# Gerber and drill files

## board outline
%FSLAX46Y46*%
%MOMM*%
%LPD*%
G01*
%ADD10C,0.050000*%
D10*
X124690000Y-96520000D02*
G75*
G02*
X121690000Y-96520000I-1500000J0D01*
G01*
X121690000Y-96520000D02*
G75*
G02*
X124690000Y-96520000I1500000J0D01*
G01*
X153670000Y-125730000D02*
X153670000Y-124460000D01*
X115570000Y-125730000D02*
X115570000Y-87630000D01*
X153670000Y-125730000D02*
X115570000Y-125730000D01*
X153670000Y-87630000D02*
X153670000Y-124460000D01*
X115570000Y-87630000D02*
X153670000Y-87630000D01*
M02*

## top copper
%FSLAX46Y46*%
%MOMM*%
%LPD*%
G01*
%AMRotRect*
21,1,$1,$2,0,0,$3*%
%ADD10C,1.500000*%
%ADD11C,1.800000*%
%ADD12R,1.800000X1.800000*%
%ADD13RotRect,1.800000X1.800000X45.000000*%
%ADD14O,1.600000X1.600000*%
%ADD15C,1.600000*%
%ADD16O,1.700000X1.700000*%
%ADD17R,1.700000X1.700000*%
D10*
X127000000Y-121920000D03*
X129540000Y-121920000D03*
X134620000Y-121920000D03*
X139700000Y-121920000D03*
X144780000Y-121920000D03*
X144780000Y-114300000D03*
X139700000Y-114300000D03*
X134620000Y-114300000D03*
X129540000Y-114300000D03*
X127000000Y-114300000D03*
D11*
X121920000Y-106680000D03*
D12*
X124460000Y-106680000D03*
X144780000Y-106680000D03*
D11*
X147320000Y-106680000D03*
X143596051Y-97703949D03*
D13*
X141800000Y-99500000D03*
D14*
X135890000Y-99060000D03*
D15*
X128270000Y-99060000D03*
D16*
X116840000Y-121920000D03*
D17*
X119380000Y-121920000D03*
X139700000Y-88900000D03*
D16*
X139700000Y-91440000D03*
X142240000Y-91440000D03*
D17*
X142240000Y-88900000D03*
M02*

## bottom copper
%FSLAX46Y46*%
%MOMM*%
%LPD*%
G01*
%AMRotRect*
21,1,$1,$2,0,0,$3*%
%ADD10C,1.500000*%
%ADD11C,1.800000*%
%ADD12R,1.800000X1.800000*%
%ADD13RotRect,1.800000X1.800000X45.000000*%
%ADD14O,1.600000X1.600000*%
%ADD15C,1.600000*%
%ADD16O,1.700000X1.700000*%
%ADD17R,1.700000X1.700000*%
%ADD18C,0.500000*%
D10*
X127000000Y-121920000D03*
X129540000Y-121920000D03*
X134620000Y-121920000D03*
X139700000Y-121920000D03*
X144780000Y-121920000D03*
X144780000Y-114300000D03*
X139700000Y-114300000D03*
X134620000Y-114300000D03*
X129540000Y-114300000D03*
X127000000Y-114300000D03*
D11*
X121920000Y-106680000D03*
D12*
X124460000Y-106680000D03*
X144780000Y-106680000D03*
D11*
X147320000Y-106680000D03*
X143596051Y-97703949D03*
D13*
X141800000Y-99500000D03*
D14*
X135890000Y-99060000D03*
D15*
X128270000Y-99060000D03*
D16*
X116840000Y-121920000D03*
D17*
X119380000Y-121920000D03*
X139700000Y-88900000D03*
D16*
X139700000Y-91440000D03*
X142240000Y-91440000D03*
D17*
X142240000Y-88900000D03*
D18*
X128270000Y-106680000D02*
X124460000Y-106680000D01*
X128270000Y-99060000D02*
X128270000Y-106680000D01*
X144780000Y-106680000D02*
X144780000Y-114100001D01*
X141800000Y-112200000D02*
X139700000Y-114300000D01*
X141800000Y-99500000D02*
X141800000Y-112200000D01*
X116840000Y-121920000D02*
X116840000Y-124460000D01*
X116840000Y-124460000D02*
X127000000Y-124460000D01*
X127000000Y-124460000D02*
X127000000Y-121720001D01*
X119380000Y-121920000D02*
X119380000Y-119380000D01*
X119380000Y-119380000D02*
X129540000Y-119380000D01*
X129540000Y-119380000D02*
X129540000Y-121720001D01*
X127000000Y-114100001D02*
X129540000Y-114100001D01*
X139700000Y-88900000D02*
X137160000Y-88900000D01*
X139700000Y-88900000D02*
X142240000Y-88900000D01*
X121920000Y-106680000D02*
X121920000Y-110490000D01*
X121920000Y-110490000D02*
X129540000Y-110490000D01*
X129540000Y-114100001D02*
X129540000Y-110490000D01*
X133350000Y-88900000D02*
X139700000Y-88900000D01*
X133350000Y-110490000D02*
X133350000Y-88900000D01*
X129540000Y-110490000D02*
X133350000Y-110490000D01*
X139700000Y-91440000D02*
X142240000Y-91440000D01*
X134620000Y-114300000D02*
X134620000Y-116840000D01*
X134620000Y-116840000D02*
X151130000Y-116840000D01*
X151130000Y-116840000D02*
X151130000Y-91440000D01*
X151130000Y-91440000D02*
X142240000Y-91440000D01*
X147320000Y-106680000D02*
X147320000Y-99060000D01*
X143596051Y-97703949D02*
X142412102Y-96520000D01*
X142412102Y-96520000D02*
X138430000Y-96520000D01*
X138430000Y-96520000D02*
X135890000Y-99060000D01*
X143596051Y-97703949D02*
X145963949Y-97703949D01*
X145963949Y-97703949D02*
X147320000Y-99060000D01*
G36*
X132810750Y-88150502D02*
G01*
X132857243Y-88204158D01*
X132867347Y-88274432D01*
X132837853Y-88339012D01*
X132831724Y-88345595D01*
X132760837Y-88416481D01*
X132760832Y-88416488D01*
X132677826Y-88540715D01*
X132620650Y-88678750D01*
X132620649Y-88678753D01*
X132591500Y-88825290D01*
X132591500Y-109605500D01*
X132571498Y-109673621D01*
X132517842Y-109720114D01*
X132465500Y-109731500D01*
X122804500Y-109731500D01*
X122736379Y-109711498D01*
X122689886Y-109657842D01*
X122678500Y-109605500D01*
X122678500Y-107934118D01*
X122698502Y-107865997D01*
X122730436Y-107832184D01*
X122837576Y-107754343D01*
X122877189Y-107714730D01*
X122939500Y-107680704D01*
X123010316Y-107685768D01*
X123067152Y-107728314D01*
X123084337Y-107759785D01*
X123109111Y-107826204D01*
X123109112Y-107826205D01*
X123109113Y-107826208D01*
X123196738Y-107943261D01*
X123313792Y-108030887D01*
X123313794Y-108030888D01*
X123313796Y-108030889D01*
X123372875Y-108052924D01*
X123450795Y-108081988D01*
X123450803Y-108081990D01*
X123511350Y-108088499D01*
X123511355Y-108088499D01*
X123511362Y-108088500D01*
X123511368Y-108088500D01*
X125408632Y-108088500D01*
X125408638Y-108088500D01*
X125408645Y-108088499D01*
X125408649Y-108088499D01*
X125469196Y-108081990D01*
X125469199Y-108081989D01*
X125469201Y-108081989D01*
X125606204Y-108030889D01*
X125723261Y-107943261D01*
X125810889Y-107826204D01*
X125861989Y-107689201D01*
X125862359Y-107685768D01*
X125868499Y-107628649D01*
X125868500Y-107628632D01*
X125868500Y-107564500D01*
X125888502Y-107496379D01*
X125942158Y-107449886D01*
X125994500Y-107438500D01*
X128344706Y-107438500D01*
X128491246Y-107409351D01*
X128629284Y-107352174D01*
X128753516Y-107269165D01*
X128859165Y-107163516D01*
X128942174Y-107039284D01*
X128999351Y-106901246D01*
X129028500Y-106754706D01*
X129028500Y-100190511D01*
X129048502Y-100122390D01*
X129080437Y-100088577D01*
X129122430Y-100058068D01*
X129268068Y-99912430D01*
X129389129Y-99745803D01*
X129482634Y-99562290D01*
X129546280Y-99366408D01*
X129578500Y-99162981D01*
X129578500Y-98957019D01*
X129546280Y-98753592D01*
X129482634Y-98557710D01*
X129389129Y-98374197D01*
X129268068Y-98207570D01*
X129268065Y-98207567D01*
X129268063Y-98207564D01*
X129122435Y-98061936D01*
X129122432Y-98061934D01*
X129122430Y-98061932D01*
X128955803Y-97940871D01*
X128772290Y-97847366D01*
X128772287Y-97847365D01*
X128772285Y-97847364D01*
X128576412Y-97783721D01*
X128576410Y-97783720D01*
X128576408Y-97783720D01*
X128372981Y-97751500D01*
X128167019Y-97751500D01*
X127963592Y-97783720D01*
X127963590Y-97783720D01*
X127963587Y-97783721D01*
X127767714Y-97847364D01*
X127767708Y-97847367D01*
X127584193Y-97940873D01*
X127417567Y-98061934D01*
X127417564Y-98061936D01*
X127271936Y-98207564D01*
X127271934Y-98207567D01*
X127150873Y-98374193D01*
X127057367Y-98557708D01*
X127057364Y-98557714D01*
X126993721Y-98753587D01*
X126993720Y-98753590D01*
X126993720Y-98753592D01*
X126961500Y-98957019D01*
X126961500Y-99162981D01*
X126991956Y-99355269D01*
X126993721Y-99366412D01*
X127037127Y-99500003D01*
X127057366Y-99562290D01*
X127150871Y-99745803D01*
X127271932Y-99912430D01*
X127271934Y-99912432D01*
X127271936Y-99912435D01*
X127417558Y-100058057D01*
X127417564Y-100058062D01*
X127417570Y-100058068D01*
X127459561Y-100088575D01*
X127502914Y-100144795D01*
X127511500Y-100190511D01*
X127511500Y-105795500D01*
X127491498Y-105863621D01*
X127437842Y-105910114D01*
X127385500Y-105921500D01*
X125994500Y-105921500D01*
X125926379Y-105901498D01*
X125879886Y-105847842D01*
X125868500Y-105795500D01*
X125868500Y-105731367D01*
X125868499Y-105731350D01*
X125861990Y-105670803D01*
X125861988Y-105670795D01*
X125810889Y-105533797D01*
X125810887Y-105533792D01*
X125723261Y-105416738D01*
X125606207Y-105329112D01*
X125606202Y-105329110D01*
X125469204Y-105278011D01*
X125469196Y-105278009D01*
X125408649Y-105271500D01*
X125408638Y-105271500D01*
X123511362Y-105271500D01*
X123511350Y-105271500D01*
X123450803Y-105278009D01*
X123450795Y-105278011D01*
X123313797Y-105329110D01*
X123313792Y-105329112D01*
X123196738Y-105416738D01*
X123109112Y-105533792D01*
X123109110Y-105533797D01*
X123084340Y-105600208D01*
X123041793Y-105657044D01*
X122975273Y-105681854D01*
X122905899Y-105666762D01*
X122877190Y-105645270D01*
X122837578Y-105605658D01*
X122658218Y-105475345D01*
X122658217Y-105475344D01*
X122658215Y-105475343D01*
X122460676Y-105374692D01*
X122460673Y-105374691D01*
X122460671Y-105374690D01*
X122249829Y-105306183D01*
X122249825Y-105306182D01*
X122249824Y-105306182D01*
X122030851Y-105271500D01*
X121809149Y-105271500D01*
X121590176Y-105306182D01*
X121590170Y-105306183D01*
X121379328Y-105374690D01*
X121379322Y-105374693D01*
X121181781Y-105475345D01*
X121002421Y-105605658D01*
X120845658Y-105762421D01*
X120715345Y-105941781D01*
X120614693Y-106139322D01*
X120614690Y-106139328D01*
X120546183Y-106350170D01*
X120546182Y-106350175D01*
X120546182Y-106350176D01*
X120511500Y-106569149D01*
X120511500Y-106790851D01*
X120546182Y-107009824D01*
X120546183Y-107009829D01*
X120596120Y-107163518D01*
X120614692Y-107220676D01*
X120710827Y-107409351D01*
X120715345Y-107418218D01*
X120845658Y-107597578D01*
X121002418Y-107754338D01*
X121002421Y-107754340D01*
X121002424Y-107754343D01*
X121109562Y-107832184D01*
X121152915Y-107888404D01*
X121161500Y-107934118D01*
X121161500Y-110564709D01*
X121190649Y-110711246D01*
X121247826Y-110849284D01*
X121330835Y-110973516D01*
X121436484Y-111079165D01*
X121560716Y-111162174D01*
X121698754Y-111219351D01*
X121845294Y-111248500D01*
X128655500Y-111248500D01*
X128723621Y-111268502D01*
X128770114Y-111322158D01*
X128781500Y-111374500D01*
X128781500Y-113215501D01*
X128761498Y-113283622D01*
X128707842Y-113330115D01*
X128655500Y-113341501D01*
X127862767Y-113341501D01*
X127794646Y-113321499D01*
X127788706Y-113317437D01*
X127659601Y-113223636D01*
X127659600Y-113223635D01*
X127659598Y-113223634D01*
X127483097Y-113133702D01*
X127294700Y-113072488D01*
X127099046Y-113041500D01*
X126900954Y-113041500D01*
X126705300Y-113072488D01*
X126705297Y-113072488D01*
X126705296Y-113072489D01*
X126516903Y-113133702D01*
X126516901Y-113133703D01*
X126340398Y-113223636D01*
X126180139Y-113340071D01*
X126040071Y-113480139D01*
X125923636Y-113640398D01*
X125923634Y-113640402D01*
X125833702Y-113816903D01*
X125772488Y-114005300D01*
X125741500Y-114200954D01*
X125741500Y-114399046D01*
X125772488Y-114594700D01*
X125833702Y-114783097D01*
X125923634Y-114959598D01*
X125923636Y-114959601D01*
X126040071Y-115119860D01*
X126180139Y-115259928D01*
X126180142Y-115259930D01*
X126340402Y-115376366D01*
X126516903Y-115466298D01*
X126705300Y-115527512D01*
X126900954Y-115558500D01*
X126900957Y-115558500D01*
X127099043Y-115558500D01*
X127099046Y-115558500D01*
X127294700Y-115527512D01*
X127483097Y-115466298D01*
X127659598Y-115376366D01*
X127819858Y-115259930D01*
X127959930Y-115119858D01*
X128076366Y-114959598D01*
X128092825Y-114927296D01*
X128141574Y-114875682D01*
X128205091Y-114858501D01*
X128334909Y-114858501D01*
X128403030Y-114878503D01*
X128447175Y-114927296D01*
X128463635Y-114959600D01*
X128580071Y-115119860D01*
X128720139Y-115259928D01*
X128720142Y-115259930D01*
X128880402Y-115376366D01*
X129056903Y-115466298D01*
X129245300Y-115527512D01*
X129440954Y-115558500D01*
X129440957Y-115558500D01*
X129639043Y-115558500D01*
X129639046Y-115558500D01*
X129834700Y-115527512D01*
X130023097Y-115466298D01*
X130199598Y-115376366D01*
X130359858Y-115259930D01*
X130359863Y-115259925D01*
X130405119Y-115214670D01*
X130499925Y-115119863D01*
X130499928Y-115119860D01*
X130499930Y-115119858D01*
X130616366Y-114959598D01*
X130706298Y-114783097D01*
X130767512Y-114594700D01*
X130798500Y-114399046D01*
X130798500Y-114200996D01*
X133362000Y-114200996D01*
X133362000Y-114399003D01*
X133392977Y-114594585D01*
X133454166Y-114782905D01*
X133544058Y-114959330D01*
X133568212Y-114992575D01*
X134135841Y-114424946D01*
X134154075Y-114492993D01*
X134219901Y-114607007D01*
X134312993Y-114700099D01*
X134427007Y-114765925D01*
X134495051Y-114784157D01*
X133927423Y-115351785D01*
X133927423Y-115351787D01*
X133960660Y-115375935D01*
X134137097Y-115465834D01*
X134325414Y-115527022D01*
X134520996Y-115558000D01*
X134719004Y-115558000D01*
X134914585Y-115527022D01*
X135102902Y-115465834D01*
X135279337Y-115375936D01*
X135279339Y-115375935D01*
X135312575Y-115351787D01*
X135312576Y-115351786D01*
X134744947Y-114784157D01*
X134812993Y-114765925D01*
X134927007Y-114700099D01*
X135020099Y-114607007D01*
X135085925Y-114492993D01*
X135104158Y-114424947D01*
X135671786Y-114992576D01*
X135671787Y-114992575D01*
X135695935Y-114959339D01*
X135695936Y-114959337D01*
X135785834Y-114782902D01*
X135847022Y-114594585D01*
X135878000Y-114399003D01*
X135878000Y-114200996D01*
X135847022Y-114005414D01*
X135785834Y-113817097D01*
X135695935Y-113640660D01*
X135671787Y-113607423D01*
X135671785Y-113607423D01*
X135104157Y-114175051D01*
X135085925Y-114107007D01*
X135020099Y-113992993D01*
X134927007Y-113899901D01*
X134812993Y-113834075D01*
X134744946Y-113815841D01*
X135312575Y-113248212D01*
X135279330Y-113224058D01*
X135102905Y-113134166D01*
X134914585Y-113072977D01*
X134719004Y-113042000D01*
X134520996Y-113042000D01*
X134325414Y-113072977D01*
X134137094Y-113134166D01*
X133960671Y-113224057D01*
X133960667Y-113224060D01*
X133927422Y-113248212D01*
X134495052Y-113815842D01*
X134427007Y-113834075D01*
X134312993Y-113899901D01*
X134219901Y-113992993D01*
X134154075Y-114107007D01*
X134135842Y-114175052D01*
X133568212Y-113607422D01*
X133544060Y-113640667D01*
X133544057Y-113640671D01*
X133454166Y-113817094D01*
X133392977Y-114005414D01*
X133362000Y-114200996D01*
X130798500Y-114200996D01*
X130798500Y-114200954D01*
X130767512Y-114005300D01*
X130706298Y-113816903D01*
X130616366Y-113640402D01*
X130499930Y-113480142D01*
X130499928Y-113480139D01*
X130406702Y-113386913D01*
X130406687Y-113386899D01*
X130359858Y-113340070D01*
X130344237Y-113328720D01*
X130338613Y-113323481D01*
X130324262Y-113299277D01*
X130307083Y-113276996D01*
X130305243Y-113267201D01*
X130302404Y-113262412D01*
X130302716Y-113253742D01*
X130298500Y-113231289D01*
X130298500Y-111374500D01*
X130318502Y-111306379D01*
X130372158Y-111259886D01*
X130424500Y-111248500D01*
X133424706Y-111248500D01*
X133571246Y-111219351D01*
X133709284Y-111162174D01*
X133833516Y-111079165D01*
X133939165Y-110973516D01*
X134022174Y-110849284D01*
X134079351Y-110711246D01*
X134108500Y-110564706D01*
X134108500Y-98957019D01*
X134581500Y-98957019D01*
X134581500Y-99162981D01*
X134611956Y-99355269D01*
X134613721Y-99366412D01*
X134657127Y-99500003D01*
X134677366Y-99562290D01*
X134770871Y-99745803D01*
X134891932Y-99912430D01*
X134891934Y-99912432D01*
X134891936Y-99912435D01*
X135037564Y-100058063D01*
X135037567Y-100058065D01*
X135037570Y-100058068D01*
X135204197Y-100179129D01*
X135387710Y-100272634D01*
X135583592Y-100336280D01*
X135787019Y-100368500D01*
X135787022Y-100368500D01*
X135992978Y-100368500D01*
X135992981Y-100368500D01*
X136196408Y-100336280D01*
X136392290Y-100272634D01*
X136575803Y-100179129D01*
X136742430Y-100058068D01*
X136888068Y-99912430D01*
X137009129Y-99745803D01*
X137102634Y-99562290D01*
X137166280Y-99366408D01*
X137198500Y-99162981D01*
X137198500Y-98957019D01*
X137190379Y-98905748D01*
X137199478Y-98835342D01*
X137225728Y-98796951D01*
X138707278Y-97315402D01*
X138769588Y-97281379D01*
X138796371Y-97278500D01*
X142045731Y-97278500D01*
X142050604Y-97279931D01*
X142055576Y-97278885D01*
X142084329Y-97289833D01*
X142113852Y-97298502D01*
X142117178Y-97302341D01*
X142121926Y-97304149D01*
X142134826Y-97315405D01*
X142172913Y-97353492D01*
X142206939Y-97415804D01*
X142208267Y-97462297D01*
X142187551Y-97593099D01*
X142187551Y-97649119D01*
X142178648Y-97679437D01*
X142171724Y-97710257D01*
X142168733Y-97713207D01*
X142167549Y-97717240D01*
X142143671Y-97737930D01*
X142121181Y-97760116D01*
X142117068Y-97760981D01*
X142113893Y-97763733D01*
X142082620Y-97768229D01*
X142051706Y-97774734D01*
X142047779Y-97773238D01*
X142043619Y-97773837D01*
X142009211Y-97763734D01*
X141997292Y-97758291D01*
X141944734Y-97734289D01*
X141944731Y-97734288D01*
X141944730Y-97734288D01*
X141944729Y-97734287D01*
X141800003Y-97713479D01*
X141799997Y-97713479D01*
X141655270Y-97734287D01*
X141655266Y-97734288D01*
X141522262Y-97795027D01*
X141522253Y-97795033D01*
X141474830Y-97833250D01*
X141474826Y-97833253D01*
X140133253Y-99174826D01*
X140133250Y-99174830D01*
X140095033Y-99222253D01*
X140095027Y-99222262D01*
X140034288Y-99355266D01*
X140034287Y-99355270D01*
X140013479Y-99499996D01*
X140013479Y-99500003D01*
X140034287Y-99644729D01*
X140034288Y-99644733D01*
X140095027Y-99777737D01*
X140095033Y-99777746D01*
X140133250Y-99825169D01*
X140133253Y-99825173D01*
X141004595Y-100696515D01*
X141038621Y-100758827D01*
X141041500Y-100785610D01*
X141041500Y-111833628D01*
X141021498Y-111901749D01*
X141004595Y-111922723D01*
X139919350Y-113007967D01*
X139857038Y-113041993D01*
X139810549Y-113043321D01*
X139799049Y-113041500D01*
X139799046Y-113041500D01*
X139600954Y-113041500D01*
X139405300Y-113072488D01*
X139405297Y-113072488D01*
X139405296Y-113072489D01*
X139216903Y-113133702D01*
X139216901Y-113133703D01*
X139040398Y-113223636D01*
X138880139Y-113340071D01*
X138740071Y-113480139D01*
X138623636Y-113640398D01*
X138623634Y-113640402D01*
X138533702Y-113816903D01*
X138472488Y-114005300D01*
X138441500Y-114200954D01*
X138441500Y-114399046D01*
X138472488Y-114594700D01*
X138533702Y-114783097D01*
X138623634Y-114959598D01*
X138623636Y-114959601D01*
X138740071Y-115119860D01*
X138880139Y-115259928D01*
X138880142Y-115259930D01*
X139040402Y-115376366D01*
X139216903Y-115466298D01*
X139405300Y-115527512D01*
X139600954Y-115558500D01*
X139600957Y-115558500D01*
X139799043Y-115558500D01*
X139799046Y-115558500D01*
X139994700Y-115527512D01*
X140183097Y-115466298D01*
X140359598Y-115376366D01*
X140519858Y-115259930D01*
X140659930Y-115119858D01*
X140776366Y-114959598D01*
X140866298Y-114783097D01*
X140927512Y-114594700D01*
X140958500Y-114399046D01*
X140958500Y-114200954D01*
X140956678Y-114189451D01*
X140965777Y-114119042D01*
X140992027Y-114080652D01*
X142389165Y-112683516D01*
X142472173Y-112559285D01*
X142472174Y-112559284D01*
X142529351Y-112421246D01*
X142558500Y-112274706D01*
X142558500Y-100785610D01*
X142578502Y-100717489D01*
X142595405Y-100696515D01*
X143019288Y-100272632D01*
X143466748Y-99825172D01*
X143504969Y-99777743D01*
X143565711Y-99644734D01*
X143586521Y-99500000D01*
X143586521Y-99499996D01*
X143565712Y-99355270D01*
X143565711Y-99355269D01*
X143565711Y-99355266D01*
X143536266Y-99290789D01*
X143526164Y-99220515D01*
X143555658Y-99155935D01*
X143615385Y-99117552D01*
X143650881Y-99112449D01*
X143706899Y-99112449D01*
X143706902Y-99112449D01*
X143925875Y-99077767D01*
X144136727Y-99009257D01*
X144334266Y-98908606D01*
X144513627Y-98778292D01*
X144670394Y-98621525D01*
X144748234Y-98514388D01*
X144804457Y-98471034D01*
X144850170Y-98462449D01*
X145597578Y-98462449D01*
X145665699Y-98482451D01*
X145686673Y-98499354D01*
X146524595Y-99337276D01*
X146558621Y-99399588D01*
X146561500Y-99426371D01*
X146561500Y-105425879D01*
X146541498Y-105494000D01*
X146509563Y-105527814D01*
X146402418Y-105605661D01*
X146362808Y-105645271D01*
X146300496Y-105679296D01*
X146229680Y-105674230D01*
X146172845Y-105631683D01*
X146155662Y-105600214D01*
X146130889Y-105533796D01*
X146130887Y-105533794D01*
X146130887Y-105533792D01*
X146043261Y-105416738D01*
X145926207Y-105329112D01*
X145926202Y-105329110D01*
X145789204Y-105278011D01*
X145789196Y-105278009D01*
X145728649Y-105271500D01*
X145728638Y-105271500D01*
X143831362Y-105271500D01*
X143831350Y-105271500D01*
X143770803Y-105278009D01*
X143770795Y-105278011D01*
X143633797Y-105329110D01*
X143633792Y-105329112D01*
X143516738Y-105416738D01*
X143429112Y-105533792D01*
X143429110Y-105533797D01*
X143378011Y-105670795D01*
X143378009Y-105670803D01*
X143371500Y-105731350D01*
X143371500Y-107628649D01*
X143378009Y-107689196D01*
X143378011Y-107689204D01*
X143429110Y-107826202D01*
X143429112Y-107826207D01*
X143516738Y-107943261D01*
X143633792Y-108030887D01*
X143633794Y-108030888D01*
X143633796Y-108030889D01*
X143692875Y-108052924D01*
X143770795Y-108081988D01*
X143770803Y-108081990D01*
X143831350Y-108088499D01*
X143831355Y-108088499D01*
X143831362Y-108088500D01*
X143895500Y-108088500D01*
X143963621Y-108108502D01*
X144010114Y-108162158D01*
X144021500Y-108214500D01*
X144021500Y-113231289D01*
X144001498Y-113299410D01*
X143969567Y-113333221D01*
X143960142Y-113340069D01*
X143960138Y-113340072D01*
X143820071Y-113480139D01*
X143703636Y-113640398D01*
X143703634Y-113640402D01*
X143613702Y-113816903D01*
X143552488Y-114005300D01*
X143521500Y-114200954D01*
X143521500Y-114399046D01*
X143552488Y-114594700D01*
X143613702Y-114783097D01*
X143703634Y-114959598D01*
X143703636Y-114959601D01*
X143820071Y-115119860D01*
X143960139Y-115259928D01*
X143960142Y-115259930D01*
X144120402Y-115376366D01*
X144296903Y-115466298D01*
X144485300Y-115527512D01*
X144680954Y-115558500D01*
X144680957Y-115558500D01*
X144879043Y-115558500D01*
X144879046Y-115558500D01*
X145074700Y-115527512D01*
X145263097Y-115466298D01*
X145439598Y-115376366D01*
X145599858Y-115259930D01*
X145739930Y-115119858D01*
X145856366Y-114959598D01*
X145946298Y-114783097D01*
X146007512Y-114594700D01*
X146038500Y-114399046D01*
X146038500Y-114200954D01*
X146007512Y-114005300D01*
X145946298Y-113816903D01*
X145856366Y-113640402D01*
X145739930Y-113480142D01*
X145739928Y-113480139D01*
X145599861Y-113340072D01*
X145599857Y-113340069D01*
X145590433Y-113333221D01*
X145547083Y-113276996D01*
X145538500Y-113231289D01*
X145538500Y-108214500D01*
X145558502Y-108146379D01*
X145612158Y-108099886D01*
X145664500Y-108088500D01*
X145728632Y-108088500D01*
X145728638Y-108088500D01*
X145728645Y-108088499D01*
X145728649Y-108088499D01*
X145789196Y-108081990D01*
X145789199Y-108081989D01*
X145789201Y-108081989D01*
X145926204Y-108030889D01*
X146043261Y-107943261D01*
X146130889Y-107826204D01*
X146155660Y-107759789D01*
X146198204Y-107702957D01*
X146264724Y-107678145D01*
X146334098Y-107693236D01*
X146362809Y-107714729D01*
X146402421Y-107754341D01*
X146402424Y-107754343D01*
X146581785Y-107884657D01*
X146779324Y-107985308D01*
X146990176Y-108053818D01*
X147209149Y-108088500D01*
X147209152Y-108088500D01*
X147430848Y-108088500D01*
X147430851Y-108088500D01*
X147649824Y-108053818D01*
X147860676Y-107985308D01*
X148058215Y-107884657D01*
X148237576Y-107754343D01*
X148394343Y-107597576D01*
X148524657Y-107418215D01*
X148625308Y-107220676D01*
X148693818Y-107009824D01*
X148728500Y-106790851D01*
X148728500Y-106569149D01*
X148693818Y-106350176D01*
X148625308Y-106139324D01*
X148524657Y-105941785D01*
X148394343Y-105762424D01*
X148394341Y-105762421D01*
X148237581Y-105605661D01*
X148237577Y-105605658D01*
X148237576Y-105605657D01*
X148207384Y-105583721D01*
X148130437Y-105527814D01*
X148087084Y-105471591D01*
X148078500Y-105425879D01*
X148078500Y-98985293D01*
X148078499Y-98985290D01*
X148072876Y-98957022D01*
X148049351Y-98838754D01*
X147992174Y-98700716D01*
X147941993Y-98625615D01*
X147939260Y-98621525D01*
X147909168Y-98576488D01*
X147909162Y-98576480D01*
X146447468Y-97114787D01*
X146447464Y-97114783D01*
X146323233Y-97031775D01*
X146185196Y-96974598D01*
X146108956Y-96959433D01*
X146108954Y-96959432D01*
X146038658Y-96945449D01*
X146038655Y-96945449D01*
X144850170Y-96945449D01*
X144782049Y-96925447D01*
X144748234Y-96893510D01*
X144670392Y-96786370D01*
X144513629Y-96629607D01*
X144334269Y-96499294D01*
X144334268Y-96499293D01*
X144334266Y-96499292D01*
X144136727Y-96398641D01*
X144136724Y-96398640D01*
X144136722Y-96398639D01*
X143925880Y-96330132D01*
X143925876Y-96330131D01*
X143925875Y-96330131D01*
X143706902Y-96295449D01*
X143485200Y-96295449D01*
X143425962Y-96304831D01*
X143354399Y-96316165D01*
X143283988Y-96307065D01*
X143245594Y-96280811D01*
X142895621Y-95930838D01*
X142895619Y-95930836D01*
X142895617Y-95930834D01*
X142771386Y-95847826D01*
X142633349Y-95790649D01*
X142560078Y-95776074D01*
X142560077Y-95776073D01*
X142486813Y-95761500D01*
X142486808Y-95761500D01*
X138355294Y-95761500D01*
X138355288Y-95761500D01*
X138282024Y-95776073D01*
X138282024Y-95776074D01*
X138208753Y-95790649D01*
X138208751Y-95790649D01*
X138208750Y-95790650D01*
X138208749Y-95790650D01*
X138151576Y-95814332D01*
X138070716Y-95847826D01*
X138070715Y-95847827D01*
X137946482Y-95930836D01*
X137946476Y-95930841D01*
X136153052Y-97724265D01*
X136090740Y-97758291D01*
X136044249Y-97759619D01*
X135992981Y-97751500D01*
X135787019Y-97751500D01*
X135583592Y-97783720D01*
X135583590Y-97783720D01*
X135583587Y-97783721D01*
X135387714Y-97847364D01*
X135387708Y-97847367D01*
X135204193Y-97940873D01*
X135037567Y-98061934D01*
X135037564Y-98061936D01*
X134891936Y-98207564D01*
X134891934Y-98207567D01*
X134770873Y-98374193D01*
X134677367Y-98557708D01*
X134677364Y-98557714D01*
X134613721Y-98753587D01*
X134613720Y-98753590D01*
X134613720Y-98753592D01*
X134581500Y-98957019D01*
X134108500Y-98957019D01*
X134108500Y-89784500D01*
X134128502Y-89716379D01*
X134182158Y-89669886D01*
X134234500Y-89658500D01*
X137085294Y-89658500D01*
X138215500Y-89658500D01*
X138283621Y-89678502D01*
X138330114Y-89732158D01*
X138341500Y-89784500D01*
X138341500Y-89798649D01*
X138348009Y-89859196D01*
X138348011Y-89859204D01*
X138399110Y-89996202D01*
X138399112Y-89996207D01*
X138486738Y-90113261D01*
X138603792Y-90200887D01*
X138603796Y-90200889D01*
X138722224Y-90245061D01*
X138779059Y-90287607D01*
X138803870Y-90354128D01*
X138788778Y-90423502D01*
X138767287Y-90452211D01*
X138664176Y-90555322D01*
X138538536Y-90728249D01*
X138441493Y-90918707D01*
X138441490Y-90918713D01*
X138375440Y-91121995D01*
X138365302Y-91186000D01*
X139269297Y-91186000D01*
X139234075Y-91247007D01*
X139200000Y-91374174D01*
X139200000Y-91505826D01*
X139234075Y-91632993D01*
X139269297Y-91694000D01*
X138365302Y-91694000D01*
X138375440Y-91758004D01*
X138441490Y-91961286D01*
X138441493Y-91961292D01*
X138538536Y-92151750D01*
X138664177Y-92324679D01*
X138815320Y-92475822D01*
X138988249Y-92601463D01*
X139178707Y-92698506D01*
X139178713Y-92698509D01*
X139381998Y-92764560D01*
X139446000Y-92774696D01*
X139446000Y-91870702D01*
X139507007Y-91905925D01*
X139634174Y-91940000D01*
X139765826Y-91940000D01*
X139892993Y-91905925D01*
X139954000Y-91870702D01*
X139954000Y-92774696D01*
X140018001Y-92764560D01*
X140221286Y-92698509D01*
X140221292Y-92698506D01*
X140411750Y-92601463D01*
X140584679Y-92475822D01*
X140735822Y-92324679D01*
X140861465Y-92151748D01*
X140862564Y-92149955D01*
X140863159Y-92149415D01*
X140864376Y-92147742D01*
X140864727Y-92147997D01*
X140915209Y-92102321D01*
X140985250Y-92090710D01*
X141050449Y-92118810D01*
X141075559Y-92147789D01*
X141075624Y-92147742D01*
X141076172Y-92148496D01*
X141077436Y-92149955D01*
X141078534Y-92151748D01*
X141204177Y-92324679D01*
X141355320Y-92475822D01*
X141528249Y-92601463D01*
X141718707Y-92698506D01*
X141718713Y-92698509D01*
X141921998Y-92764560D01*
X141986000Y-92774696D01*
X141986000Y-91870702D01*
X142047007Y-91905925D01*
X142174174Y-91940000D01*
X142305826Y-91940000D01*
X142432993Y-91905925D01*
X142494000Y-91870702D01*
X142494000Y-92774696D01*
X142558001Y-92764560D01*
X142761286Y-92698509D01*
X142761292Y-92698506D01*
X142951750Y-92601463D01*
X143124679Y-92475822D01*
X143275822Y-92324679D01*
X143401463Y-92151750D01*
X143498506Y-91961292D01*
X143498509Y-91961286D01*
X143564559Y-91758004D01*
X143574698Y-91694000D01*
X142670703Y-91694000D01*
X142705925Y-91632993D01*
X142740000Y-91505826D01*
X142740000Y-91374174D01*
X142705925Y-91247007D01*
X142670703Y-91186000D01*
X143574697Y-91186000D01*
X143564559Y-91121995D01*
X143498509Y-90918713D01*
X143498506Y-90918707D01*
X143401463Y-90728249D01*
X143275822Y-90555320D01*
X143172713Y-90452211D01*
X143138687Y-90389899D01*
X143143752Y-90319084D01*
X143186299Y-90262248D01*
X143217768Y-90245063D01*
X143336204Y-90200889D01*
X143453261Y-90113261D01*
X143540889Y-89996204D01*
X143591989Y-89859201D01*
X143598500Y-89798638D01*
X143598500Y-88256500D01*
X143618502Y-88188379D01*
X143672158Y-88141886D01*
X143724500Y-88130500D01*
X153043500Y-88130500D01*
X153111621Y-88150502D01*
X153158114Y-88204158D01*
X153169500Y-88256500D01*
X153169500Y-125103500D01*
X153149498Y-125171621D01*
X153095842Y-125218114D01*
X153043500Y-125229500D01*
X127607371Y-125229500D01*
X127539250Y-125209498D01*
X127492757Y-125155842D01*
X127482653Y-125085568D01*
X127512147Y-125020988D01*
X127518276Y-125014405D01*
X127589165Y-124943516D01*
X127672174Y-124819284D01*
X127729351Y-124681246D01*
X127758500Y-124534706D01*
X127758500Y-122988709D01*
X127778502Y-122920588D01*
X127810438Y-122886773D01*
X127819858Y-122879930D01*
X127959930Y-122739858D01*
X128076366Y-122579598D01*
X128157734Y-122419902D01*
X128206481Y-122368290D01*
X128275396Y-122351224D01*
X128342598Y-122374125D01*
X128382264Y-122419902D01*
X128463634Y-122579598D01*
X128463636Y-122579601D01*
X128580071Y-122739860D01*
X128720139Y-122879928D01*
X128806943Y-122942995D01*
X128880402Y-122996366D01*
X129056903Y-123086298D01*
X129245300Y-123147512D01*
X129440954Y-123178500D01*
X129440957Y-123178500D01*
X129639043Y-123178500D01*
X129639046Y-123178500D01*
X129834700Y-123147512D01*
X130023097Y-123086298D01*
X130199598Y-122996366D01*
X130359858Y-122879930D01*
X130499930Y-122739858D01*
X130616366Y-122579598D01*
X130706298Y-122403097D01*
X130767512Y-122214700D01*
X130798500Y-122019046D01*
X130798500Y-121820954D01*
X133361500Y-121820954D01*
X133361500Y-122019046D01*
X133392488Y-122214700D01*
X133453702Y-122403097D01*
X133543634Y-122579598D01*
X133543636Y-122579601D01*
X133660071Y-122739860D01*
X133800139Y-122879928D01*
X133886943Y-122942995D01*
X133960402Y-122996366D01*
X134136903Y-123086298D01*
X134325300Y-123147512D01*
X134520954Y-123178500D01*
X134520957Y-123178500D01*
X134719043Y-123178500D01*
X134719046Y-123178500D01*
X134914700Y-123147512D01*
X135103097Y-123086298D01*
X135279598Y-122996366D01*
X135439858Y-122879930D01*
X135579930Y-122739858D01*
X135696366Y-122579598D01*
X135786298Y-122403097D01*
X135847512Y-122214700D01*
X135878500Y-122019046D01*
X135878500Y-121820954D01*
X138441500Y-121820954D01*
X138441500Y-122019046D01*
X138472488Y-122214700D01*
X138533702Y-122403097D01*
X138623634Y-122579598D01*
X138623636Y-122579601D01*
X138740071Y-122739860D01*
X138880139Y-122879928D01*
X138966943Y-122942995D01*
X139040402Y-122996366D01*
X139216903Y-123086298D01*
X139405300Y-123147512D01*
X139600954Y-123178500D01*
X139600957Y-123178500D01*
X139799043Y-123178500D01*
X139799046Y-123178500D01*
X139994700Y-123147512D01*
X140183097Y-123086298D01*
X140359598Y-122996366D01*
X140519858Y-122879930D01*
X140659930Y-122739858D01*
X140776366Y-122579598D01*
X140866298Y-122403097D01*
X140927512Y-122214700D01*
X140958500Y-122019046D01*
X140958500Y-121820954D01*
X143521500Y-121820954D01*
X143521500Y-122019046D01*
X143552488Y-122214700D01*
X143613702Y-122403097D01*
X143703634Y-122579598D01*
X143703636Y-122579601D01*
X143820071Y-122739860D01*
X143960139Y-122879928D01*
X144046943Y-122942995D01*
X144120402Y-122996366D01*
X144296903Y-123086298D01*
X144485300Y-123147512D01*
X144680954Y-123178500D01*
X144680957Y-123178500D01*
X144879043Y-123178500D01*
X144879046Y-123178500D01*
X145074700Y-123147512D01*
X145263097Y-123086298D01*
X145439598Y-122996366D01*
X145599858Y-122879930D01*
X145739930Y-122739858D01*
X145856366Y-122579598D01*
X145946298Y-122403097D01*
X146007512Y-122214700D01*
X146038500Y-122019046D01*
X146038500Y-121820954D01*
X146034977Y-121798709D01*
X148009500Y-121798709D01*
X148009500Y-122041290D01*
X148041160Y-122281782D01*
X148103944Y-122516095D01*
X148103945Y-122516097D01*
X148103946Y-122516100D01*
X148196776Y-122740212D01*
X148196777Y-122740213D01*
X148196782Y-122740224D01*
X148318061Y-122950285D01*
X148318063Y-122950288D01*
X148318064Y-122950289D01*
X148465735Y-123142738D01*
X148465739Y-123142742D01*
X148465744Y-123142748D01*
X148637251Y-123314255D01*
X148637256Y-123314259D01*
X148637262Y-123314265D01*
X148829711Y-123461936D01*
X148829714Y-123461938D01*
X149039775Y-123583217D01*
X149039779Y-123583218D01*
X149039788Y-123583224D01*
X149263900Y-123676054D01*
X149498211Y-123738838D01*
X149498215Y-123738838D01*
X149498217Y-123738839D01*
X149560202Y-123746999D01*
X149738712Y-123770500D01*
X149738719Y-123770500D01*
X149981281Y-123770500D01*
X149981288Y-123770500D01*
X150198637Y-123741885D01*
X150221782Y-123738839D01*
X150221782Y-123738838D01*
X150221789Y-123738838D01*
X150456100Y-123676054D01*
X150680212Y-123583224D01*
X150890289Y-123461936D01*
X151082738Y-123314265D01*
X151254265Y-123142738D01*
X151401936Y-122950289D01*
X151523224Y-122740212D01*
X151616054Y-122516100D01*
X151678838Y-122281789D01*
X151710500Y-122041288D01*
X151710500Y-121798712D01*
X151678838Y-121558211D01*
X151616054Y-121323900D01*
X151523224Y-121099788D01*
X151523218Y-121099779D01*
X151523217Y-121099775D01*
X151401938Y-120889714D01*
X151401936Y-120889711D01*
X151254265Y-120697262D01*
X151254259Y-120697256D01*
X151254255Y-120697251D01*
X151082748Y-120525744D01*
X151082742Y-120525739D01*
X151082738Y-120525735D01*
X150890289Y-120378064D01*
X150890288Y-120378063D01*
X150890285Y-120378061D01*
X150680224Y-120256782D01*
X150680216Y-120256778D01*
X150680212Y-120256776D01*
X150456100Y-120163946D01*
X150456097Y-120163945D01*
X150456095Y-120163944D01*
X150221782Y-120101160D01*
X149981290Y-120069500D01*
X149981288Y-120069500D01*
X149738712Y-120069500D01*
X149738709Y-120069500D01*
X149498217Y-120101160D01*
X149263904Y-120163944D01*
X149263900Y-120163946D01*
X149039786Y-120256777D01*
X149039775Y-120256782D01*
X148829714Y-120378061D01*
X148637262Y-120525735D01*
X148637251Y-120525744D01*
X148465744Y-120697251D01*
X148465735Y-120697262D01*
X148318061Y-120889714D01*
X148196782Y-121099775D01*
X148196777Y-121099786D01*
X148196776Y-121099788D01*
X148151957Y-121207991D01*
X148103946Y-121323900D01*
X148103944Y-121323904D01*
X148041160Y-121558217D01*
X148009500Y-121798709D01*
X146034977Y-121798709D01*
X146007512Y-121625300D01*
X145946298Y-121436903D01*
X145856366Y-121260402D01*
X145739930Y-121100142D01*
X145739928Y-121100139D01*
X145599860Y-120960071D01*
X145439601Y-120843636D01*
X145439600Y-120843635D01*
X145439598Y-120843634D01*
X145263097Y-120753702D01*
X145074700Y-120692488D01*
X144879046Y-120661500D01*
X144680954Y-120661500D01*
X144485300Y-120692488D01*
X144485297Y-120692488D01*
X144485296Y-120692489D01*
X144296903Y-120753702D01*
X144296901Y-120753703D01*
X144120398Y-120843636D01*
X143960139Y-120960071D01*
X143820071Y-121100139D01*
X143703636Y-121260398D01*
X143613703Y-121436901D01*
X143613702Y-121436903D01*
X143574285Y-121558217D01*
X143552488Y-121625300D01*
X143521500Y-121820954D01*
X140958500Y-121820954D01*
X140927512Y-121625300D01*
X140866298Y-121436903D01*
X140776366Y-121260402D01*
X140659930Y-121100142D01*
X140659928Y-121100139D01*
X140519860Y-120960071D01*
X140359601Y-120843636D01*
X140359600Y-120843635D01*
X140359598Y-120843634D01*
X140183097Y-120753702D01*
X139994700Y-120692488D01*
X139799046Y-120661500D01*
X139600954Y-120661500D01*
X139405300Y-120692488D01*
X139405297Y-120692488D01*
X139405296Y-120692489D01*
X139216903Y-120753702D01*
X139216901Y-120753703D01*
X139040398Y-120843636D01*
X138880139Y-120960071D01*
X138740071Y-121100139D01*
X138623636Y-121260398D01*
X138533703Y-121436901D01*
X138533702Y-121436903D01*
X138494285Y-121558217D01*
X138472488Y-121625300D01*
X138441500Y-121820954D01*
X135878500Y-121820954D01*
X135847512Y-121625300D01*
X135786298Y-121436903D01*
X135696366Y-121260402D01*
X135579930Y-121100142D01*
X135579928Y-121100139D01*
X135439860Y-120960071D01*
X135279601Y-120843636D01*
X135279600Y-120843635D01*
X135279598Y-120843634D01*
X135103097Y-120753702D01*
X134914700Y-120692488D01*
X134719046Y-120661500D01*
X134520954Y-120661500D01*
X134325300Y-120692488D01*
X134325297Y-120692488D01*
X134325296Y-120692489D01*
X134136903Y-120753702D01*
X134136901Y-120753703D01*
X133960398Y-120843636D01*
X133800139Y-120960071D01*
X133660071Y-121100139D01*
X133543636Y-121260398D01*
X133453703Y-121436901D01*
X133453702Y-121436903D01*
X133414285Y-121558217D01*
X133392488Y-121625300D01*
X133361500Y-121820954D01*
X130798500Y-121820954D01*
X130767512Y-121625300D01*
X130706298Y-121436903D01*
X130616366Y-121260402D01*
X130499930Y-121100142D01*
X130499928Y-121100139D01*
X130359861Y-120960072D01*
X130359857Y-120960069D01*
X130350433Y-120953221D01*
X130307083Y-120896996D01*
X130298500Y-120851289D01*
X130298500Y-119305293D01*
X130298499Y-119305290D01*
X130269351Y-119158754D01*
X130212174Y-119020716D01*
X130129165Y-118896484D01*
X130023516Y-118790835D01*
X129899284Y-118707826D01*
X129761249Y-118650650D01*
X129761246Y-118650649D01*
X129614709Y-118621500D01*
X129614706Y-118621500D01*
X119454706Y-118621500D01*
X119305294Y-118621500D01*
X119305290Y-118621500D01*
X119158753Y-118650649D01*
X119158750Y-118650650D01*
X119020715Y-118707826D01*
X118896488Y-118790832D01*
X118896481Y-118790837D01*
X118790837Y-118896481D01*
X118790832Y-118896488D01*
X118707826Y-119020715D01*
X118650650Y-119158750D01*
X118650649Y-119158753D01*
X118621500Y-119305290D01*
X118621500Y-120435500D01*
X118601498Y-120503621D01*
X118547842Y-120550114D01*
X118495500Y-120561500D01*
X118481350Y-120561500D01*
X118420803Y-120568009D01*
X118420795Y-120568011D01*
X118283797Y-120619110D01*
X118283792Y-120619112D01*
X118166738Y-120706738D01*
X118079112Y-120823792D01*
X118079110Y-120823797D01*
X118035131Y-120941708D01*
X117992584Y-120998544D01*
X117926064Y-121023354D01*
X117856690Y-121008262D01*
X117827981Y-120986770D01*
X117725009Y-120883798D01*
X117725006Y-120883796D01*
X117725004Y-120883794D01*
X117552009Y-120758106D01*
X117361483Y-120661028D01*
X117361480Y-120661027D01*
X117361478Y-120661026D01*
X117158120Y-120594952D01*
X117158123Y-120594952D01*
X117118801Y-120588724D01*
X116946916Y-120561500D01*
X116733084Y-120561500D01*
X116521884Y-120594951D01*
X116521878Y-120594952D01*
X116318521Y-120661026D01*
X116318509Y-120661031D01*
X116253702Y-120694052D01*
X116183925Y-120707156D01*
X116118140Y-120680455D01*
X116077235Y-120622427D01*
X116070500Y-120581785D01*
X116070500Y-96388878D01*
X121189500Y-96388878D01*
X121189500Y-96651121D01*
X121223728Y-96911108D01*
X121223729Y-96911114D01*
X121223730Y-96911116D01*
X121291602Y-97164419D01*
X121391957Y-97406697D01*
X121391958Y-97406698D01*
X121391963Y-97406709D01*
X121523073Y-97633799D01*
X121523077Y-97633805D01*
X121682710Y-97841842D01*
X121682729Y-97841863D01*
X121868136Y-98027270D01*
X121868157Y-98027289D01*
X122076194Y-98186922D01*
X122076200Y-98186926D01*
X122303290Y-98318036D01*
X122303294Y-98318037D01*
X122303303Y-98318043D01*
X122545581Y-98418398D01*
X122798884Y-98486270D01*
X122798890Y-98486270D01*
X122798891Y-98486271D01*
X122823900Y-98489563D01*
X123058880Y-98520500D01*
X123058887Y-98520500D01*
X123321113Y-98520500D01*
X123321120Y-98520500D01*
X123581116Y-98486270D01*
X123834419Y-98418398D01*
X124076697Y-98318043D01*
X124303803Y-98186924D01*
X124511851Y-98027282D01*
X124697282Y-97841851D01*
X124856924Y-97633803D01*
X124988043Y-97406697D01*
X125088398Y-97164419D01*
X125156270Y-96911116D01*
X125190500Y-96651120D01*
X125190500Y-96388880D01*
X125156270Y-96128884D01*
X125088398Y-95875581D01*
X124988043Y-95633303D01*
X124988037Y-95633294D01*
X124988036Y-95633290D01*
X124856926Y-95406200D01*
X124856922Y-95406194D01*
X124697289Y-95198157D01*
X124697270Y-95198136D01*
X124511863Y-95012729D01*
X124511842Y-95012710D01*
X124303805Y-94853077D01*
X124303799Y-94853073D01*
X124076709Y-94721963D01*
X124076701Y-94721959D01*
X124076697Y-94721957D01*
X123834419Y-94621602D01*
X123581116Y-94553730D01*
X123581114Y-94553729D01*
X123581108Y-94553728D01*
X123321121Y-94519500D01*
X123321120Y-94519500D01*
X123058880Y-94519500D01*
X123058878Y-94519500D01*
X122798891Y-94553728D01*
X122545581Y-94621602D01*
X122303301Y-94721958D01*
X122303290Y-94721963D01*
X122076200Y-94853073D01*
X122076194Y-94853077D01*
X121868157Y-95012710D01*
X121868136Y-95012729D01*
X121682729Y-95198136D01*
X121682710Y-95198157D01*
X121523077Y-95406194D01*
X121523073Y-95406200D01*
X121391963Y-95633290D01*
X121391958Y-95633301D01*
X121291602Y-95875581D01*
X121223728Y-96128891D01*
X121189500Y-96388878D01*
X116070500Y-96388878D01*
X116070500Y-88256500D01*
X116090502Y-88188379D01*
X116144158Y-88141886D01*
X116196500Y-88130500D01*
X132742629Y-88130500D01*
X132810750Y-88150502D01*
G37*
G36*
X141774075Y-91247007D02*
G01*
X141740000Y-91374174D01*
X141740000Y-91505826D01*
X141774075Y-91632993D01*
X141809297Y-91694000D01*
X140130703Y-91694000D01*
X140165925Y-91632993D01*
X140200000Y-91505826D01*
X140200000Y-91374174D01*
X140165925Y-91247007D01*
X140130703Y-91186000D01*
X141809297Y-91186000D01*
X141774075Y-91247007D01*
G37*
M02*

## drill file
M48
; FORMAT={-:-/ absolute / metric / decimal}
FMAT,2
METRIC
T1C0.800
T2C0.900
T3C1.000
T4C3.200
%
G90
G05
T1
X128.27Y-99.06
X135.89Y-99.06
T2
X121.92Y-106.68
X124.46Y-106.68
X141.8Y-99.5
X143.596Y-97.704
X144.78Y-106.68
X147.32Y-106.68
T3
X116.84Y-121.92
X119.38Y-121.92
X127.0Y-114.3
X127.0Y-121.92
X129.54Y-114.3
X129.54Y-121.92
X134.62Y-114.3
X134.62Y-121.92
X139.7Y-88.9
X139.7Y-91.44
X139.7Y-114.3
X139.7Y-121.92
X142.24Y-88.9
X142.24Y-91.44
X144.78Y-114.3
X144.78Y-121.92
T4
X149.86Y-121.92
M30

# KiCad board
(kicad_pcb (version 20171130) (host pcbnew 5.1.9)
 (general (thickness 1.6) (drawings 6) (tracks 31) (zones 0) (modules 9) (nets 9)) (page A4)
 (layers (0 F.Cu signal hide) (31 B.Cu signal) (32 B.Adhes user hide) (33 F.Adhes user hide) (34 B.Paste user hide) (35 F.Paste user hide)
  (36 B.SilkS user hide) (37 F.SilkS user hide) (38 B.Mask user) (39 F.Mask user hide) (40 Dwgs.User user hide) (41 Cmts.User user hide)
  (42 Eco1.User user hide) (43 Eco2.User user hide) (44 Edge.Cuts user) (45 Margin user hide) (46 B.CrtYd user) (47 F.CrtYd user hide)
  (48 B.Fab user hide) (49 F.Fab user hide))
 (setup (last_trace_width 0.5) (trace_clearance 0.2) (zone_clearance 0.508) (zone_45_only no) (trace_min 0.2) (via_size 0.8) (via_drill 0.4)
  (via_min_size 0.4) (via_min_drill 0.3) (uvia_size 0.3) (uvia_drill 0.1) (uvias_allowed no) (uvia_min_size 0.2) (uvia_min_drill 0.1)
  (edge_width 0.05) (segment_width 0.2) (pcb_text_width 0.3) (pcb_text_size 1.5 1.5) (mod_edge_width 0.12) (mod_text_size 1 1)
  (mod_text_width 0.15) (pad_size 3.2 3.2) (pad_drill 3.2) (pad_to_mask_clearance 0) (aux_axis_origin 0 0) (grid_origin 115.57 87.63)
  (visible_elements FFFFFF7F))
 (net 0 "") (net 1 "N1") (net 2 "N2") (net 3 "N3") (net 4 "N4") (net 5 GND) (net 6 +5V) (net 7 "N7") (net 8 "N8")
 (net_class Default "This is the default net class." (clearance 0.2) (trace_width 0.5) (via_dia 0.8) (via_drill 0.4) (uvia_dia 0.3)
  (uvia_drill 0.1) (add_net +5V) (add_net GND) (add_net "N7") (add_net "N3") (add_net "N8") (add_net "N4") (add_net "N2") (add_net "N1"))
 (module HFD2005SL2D (layer F.Cu) (at 127 121.92)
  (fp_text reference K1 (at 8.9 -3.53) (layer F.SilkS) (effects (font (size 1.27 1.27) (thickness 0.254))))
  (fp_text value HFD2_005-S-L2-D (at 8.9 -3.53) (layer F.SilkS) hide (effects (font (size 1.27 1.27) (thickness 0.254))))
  (pad 1 thru_hole circle (at 0 0 90) (size 1.5 1.5) (drill 1) (layers *.Cu *.Mask F.SilkS) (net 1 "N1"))
  (pad 2 thru_hole circle (at 2.54 0 90) (size 1.5 1.5) (drill 1) (layers *.Cu *.Mask F.SilkS) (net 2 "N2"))
  (pad 4 thru_hole circle (at 7.62 0 90) (size 1.5 1.5) (drill 1) (layers *.Cu *.Mask F.SilkS))
  (pad 6 thru_hole circle (at 12.7 0 90) (size 1.5 1.5) (drill 1) (layers *.Cu *.Mask F.SilkS))
  (pad 8 thru_hole circle (at 17.78 0 90) (size 1.5 1.5) (drill 1) (layers *.Cu *.Mask F.SilkS))
  (pad 9 thru_hole circle (at 17.78 -7.62 90) (size 1.5 1.5) (drill 1) (layers *.Cu *.Mask F.SilkS) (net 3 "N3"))
  (pad 11 thru_hole circle (at 12.7 -7.62 90) (size 1.5 1.5) (drill 1) (layers *.Cu *.Mask F.SilkS) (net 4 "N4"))
  (pad 13 thru_hole circle (at 7.62 -7.62 90) (size 1.5 1.5) (drill 1) (layers *.Cu *.Mask F.SilkS) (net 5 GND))
  (pad 15 thru_hole circle (at 2.54 -7.62 90) (size 1.5 1.5) (drill 1) (layers *.Cu *.Mask F.SilkS) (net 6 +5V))
  (pad 16 thru_hole circle (at 0 -7.62 90) (size 1.5 1.5) (drill 1) (layers *.Cu *.Mask F.SilkS) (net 6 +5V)))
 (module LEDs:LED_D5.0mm (layer F.Cu) (at 124.46 106.68 180)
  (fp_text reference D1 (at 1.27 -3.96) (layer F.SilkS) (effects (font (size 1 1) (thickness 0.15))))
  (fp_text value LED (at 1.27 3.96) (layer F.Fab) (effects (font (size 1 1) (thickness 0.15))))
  (pad 2 thru_hole circle (at 2.54 0 180) (size 1.8 1.8) (drill 0.9) (layers *.Cu *.Mask) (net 6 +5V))
  (pad 1 thru_hole rect (at 0 0 180) (size 1.8 1.8) (drill 0.9) (layers *.Cu *.Mask) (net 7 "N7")))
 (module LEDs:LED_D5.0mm (layer F.Cu) (at 144.78 106.68)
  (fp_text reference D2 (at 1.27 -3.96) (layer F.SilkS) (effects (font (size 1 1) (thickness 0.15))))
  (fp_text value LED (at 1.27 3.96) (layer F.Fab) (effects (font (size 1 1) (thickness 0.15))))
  (pad 1 thru_hole rect (at 0 0) (size 1.8 1.8) (drill 0.9) (layers *.Cu *.Mask) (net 3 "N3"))
  (pad 2 thru_hole circle (at 2.54 0) (size 1.8 1.8) (drill 0.9) (layers *.Cu *.Mask) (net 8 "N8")))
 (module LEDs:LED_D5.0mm (layer F.Cu) (at 141.8 99.5 45)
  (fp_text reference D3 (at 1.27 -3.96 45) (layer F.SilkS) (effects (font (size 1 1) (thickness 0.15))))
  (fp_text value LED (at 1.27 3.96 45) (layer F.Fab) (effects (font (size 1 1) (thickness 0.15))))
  (pad 2 thru_hole circle (at 2.54 0 45) (size 1.8 1.8) (drill 0.9) (layers *.Cu *.Mask) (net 8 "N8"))
  (pad 1 thru_hole rect (at 0 0 45) (size 1.8 1.8) (drill 0.9) (layers *.Cu *.Mask) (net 4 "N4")))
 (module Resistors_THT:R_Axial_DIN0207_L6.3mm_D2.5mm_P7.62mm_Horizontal (layer F.Cu) (at 128.27 99.06)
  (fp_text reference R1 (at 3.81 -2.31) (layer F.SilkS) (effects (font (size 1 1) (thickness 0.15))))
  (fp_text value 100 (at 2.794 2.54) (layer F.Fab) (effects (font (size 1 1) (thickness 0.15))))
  (pad 2 thru_hole oval (at 7.62 0) (size 1.6 1.6) (drill 0.8) (layers *.Cu *.Mask) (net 8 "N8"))
  (pad 1 thru_hole circle (at 0 0) (size 1.6 1.6) (drill 0.8) (layers *.Cu *.Mask) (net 7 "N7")))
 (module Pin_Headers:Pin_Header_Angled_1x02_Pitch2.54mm (layer B.Cu) (at 119.38 121.92 90)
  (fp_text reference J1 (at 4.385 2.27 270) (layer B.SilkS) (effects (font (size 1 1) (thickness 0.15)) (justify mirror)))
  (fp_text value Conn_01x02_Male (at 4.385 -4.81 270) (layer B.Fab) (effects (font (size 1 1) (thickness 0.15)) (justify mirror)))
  (pad 2 thru_hole oval (at 0 -2.54 90) (size 1.7 1.7) (drill 1) (layers *.Cu *.Mask) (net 1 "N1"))
  (pad 1 thru_hole rect (at 0 0 90) (size 1.7 1.7) (drill 1) (layers *.Cu *.Mask) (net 2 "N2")))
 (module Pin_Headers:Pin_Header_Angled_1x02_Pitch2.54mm (layer B.Cu) (at 139.7 88.9 180)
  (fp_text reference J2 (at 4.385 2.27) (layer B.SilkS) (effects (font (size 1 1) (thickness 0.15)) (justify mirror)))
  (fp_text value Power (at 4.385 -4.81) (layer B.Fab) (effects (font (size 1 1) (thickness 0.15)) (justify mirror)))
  (pad 1 thru_hole rect (at 0 0 180) (size 1.7 1.7) (drill 1) (layers *.Cu *.Mask) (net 6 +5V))
  (pad 2 thru_hole oval (at 0 -2.54 180) (size 1.7 1.7) (drill 1) (layers *.Cu *.Mask) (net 5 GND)))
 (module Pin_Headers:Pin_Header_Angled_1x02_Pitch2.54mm (layer B.Cu) (at 142.24 88.9 180)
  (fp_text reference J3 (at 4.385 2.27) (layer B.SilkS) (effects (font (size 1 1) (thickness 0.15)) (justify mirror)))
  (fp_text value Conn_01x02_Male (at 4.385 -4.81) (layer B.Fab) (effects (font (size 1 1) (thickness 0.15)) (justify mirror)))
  (pad 2 thru_hole oval (at 0 -2.54 180) (size 1.7 1.7) (drill 1) (layers *.Cu *.Mask) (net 5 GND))
  (pad 1 thru_hole rect (at 0 0 180) (size 1.7 1.7) (drill 1) (layers *.Cu *.Mask) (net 6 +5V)))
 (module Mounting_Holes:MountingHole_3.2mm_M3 (layer F.Cu) (at 149.86 121.92)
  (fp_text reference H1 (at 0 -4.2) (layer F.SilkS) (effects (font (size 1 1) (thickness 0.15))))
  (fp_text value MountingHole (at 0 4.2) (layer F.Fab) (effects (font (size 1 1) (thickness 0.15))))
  (pad "" np_thru_hole circle (at 0 0) (size 3.2 3.2) (drill 3.2) (layers *.Cu *.Mask) (thermal_gap 2)))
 (gr_circle (center 123.19 96.52) (end 124.69 96.52) (layer Edge.Cuts) (width 0.05))
 (gr_line (start 153.67 125.73) (end 153.67 124.46) (layer Edge.Cuts) (width 0.05))
 (gr_line (start 115.57 125.73) (end 115.57 87.63) (layer Edge.Cuts) (width 0.05))
 (gr_line (start 153.67 125.73) (end 115.57 125.73) (layer Edge.Cuts) (width 0.05))
 (gr_line (start 153.67 87.63) (end 153.67 124.46) (layer Edge.Cuts) (width 0.05))
 (gr_line (start 115.57 87.63) (end 153.67 87.63) (layer Edge.Cuts) (width 0.05))
 (segment (start 128.27 106.68) (end 124.46 106.68) (width 0.5) (layer B.Cu) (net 7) (status 20))
 (segment (start 128.27 99.06) (end 128.27 106.68) (width 0.5) (layer B.Cu) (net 7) (status 10))
 (segment (start 144.78 106.68) (end 144.78 114.100001) (width 0.5) (layer B.Cu) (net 3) (status 30))
 (segment (start 141.8 112.2) (end 139.7 114.3) (width 0.5) (layer B.Cu) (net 4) (status 20))
 (segment (start 141.8 99.5) (end 141.8 112.2) (width 0.5) (layer B.Cu) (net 4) (status 10))
 (segment (start 116.84 121.92) (end 116.84 124.46) (width 0.5) (layer B.Cu) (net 1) (status 10))
 (segment (start 116.84 124.46) (end 127 124.46) (width 0.5) (layer B.Cu) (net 1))
 (segment (start 127 124.46) (end 127 121.720001) (width 0.5) (layer B.Cu) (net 1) (status 20))
 (segment (start 119.38 121.92) (end 119.38 119.38) (width 0.5) (layer B.Cu) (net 2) (status 10))
 (segment (start 119.38 119.38) (end 129.54 119.38) (width 0.5) (layer B.Cu) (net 2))
 (segment (start 129.54 119.38) (end 129.54 121.720001) (width 0.5) (layer B.Cu) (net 2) (status 20))
 (segment (start 127 114.100001) (end 129.54 114.100001) (width 0.5) (layer B.Cu) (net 6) (status 30))
 (segment (start 139.7 88.9) (end 137.16 88.9) (width 0.5) (layer B.Cu) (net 6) (status 10))
 (segment (start 139.7 88.9) (end 142.24 88.9) (width 0.5) (layer B.Cu) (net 6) (status 30))
 (segment (start 121.92 106.68) (end 121.92 110.49) (width 0.5) (layer B.Cu) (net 6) (status 10))
 (segment (start 121.92 110.49) (end 129.54 110.49) (width 0.5) (layer B.Cu) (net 6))
 (segment (start 129.54 114.100001) (end 129.54 110.49) (width 0.5) (layer B.Cu) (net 6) (status 10))
 (segment (start 133.35 88.9) (end 139.7 88.9) (width 0.5) (layer B.Cu) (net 6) (status 20))
 (segment (start 133.35 110.49) (end 133.35 88.9) (width 0.5) (layer B.Cu) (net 6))
 (segment (start 129.54 110.49) (end 133.35 110.49) (width 0.5) (layer B.Cu) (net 6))
 (segment (start 139.7 91.44) (end 142.24 91.44) (width 0.5) (layer B.Cu) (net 5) (status 30))
 (segment (start 134.62 114.3) (end 134.62 116.84) (width 0.5) (layer B.Cu) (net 5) (status 10))
 (segment (start 134.62 116.84) (end 151.13 116.84) (width 0.5) (layer B.Cu) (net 5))
 (segment (start 151.13 116.84) (end 151.13 91.44) (width 0.5) (layer B.Cu) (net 5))
 (segment (start 151.13 91.44) (end 142.24 91.44) (width 0.5) (layer B.Cu) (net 5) (status 20))
 (segment (start 147.32 106.68) (end 147.32 99.06) (width 0.5) (layer B.Cu) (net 8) (status 10))
 (segment (start 143.596051 97.703949) (end 142.412102 96.52) (width 0.5) (layer B.Cu) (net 8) (status 10))
 (segment (start 142.412102 96.52) (end 138.43 96.52) (width 0.5) (layer B.Cu) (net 8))
 (segment (start 138.43 96.52) (end 135.89 99.06) (width 0.5) (layer B.Cu) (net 8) (status 20))
 (segment (start 143.596051 97.703949) (end 145.963949 97.703949) (width 0.5) (layer B.Cu) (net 8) (status 10))
 (segment (start 145.963949 97.703949) (end 147.32 99.06) (width 0.5) (layer B.Cu) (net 8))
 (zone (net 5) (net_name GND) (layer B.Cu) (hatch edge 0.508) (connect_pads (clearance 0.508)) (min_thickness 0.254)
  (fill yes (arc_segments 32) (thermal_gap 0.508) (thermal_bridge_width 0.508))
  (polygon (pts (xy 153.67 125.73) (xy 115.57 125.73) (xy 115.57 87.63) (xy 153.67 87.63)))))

